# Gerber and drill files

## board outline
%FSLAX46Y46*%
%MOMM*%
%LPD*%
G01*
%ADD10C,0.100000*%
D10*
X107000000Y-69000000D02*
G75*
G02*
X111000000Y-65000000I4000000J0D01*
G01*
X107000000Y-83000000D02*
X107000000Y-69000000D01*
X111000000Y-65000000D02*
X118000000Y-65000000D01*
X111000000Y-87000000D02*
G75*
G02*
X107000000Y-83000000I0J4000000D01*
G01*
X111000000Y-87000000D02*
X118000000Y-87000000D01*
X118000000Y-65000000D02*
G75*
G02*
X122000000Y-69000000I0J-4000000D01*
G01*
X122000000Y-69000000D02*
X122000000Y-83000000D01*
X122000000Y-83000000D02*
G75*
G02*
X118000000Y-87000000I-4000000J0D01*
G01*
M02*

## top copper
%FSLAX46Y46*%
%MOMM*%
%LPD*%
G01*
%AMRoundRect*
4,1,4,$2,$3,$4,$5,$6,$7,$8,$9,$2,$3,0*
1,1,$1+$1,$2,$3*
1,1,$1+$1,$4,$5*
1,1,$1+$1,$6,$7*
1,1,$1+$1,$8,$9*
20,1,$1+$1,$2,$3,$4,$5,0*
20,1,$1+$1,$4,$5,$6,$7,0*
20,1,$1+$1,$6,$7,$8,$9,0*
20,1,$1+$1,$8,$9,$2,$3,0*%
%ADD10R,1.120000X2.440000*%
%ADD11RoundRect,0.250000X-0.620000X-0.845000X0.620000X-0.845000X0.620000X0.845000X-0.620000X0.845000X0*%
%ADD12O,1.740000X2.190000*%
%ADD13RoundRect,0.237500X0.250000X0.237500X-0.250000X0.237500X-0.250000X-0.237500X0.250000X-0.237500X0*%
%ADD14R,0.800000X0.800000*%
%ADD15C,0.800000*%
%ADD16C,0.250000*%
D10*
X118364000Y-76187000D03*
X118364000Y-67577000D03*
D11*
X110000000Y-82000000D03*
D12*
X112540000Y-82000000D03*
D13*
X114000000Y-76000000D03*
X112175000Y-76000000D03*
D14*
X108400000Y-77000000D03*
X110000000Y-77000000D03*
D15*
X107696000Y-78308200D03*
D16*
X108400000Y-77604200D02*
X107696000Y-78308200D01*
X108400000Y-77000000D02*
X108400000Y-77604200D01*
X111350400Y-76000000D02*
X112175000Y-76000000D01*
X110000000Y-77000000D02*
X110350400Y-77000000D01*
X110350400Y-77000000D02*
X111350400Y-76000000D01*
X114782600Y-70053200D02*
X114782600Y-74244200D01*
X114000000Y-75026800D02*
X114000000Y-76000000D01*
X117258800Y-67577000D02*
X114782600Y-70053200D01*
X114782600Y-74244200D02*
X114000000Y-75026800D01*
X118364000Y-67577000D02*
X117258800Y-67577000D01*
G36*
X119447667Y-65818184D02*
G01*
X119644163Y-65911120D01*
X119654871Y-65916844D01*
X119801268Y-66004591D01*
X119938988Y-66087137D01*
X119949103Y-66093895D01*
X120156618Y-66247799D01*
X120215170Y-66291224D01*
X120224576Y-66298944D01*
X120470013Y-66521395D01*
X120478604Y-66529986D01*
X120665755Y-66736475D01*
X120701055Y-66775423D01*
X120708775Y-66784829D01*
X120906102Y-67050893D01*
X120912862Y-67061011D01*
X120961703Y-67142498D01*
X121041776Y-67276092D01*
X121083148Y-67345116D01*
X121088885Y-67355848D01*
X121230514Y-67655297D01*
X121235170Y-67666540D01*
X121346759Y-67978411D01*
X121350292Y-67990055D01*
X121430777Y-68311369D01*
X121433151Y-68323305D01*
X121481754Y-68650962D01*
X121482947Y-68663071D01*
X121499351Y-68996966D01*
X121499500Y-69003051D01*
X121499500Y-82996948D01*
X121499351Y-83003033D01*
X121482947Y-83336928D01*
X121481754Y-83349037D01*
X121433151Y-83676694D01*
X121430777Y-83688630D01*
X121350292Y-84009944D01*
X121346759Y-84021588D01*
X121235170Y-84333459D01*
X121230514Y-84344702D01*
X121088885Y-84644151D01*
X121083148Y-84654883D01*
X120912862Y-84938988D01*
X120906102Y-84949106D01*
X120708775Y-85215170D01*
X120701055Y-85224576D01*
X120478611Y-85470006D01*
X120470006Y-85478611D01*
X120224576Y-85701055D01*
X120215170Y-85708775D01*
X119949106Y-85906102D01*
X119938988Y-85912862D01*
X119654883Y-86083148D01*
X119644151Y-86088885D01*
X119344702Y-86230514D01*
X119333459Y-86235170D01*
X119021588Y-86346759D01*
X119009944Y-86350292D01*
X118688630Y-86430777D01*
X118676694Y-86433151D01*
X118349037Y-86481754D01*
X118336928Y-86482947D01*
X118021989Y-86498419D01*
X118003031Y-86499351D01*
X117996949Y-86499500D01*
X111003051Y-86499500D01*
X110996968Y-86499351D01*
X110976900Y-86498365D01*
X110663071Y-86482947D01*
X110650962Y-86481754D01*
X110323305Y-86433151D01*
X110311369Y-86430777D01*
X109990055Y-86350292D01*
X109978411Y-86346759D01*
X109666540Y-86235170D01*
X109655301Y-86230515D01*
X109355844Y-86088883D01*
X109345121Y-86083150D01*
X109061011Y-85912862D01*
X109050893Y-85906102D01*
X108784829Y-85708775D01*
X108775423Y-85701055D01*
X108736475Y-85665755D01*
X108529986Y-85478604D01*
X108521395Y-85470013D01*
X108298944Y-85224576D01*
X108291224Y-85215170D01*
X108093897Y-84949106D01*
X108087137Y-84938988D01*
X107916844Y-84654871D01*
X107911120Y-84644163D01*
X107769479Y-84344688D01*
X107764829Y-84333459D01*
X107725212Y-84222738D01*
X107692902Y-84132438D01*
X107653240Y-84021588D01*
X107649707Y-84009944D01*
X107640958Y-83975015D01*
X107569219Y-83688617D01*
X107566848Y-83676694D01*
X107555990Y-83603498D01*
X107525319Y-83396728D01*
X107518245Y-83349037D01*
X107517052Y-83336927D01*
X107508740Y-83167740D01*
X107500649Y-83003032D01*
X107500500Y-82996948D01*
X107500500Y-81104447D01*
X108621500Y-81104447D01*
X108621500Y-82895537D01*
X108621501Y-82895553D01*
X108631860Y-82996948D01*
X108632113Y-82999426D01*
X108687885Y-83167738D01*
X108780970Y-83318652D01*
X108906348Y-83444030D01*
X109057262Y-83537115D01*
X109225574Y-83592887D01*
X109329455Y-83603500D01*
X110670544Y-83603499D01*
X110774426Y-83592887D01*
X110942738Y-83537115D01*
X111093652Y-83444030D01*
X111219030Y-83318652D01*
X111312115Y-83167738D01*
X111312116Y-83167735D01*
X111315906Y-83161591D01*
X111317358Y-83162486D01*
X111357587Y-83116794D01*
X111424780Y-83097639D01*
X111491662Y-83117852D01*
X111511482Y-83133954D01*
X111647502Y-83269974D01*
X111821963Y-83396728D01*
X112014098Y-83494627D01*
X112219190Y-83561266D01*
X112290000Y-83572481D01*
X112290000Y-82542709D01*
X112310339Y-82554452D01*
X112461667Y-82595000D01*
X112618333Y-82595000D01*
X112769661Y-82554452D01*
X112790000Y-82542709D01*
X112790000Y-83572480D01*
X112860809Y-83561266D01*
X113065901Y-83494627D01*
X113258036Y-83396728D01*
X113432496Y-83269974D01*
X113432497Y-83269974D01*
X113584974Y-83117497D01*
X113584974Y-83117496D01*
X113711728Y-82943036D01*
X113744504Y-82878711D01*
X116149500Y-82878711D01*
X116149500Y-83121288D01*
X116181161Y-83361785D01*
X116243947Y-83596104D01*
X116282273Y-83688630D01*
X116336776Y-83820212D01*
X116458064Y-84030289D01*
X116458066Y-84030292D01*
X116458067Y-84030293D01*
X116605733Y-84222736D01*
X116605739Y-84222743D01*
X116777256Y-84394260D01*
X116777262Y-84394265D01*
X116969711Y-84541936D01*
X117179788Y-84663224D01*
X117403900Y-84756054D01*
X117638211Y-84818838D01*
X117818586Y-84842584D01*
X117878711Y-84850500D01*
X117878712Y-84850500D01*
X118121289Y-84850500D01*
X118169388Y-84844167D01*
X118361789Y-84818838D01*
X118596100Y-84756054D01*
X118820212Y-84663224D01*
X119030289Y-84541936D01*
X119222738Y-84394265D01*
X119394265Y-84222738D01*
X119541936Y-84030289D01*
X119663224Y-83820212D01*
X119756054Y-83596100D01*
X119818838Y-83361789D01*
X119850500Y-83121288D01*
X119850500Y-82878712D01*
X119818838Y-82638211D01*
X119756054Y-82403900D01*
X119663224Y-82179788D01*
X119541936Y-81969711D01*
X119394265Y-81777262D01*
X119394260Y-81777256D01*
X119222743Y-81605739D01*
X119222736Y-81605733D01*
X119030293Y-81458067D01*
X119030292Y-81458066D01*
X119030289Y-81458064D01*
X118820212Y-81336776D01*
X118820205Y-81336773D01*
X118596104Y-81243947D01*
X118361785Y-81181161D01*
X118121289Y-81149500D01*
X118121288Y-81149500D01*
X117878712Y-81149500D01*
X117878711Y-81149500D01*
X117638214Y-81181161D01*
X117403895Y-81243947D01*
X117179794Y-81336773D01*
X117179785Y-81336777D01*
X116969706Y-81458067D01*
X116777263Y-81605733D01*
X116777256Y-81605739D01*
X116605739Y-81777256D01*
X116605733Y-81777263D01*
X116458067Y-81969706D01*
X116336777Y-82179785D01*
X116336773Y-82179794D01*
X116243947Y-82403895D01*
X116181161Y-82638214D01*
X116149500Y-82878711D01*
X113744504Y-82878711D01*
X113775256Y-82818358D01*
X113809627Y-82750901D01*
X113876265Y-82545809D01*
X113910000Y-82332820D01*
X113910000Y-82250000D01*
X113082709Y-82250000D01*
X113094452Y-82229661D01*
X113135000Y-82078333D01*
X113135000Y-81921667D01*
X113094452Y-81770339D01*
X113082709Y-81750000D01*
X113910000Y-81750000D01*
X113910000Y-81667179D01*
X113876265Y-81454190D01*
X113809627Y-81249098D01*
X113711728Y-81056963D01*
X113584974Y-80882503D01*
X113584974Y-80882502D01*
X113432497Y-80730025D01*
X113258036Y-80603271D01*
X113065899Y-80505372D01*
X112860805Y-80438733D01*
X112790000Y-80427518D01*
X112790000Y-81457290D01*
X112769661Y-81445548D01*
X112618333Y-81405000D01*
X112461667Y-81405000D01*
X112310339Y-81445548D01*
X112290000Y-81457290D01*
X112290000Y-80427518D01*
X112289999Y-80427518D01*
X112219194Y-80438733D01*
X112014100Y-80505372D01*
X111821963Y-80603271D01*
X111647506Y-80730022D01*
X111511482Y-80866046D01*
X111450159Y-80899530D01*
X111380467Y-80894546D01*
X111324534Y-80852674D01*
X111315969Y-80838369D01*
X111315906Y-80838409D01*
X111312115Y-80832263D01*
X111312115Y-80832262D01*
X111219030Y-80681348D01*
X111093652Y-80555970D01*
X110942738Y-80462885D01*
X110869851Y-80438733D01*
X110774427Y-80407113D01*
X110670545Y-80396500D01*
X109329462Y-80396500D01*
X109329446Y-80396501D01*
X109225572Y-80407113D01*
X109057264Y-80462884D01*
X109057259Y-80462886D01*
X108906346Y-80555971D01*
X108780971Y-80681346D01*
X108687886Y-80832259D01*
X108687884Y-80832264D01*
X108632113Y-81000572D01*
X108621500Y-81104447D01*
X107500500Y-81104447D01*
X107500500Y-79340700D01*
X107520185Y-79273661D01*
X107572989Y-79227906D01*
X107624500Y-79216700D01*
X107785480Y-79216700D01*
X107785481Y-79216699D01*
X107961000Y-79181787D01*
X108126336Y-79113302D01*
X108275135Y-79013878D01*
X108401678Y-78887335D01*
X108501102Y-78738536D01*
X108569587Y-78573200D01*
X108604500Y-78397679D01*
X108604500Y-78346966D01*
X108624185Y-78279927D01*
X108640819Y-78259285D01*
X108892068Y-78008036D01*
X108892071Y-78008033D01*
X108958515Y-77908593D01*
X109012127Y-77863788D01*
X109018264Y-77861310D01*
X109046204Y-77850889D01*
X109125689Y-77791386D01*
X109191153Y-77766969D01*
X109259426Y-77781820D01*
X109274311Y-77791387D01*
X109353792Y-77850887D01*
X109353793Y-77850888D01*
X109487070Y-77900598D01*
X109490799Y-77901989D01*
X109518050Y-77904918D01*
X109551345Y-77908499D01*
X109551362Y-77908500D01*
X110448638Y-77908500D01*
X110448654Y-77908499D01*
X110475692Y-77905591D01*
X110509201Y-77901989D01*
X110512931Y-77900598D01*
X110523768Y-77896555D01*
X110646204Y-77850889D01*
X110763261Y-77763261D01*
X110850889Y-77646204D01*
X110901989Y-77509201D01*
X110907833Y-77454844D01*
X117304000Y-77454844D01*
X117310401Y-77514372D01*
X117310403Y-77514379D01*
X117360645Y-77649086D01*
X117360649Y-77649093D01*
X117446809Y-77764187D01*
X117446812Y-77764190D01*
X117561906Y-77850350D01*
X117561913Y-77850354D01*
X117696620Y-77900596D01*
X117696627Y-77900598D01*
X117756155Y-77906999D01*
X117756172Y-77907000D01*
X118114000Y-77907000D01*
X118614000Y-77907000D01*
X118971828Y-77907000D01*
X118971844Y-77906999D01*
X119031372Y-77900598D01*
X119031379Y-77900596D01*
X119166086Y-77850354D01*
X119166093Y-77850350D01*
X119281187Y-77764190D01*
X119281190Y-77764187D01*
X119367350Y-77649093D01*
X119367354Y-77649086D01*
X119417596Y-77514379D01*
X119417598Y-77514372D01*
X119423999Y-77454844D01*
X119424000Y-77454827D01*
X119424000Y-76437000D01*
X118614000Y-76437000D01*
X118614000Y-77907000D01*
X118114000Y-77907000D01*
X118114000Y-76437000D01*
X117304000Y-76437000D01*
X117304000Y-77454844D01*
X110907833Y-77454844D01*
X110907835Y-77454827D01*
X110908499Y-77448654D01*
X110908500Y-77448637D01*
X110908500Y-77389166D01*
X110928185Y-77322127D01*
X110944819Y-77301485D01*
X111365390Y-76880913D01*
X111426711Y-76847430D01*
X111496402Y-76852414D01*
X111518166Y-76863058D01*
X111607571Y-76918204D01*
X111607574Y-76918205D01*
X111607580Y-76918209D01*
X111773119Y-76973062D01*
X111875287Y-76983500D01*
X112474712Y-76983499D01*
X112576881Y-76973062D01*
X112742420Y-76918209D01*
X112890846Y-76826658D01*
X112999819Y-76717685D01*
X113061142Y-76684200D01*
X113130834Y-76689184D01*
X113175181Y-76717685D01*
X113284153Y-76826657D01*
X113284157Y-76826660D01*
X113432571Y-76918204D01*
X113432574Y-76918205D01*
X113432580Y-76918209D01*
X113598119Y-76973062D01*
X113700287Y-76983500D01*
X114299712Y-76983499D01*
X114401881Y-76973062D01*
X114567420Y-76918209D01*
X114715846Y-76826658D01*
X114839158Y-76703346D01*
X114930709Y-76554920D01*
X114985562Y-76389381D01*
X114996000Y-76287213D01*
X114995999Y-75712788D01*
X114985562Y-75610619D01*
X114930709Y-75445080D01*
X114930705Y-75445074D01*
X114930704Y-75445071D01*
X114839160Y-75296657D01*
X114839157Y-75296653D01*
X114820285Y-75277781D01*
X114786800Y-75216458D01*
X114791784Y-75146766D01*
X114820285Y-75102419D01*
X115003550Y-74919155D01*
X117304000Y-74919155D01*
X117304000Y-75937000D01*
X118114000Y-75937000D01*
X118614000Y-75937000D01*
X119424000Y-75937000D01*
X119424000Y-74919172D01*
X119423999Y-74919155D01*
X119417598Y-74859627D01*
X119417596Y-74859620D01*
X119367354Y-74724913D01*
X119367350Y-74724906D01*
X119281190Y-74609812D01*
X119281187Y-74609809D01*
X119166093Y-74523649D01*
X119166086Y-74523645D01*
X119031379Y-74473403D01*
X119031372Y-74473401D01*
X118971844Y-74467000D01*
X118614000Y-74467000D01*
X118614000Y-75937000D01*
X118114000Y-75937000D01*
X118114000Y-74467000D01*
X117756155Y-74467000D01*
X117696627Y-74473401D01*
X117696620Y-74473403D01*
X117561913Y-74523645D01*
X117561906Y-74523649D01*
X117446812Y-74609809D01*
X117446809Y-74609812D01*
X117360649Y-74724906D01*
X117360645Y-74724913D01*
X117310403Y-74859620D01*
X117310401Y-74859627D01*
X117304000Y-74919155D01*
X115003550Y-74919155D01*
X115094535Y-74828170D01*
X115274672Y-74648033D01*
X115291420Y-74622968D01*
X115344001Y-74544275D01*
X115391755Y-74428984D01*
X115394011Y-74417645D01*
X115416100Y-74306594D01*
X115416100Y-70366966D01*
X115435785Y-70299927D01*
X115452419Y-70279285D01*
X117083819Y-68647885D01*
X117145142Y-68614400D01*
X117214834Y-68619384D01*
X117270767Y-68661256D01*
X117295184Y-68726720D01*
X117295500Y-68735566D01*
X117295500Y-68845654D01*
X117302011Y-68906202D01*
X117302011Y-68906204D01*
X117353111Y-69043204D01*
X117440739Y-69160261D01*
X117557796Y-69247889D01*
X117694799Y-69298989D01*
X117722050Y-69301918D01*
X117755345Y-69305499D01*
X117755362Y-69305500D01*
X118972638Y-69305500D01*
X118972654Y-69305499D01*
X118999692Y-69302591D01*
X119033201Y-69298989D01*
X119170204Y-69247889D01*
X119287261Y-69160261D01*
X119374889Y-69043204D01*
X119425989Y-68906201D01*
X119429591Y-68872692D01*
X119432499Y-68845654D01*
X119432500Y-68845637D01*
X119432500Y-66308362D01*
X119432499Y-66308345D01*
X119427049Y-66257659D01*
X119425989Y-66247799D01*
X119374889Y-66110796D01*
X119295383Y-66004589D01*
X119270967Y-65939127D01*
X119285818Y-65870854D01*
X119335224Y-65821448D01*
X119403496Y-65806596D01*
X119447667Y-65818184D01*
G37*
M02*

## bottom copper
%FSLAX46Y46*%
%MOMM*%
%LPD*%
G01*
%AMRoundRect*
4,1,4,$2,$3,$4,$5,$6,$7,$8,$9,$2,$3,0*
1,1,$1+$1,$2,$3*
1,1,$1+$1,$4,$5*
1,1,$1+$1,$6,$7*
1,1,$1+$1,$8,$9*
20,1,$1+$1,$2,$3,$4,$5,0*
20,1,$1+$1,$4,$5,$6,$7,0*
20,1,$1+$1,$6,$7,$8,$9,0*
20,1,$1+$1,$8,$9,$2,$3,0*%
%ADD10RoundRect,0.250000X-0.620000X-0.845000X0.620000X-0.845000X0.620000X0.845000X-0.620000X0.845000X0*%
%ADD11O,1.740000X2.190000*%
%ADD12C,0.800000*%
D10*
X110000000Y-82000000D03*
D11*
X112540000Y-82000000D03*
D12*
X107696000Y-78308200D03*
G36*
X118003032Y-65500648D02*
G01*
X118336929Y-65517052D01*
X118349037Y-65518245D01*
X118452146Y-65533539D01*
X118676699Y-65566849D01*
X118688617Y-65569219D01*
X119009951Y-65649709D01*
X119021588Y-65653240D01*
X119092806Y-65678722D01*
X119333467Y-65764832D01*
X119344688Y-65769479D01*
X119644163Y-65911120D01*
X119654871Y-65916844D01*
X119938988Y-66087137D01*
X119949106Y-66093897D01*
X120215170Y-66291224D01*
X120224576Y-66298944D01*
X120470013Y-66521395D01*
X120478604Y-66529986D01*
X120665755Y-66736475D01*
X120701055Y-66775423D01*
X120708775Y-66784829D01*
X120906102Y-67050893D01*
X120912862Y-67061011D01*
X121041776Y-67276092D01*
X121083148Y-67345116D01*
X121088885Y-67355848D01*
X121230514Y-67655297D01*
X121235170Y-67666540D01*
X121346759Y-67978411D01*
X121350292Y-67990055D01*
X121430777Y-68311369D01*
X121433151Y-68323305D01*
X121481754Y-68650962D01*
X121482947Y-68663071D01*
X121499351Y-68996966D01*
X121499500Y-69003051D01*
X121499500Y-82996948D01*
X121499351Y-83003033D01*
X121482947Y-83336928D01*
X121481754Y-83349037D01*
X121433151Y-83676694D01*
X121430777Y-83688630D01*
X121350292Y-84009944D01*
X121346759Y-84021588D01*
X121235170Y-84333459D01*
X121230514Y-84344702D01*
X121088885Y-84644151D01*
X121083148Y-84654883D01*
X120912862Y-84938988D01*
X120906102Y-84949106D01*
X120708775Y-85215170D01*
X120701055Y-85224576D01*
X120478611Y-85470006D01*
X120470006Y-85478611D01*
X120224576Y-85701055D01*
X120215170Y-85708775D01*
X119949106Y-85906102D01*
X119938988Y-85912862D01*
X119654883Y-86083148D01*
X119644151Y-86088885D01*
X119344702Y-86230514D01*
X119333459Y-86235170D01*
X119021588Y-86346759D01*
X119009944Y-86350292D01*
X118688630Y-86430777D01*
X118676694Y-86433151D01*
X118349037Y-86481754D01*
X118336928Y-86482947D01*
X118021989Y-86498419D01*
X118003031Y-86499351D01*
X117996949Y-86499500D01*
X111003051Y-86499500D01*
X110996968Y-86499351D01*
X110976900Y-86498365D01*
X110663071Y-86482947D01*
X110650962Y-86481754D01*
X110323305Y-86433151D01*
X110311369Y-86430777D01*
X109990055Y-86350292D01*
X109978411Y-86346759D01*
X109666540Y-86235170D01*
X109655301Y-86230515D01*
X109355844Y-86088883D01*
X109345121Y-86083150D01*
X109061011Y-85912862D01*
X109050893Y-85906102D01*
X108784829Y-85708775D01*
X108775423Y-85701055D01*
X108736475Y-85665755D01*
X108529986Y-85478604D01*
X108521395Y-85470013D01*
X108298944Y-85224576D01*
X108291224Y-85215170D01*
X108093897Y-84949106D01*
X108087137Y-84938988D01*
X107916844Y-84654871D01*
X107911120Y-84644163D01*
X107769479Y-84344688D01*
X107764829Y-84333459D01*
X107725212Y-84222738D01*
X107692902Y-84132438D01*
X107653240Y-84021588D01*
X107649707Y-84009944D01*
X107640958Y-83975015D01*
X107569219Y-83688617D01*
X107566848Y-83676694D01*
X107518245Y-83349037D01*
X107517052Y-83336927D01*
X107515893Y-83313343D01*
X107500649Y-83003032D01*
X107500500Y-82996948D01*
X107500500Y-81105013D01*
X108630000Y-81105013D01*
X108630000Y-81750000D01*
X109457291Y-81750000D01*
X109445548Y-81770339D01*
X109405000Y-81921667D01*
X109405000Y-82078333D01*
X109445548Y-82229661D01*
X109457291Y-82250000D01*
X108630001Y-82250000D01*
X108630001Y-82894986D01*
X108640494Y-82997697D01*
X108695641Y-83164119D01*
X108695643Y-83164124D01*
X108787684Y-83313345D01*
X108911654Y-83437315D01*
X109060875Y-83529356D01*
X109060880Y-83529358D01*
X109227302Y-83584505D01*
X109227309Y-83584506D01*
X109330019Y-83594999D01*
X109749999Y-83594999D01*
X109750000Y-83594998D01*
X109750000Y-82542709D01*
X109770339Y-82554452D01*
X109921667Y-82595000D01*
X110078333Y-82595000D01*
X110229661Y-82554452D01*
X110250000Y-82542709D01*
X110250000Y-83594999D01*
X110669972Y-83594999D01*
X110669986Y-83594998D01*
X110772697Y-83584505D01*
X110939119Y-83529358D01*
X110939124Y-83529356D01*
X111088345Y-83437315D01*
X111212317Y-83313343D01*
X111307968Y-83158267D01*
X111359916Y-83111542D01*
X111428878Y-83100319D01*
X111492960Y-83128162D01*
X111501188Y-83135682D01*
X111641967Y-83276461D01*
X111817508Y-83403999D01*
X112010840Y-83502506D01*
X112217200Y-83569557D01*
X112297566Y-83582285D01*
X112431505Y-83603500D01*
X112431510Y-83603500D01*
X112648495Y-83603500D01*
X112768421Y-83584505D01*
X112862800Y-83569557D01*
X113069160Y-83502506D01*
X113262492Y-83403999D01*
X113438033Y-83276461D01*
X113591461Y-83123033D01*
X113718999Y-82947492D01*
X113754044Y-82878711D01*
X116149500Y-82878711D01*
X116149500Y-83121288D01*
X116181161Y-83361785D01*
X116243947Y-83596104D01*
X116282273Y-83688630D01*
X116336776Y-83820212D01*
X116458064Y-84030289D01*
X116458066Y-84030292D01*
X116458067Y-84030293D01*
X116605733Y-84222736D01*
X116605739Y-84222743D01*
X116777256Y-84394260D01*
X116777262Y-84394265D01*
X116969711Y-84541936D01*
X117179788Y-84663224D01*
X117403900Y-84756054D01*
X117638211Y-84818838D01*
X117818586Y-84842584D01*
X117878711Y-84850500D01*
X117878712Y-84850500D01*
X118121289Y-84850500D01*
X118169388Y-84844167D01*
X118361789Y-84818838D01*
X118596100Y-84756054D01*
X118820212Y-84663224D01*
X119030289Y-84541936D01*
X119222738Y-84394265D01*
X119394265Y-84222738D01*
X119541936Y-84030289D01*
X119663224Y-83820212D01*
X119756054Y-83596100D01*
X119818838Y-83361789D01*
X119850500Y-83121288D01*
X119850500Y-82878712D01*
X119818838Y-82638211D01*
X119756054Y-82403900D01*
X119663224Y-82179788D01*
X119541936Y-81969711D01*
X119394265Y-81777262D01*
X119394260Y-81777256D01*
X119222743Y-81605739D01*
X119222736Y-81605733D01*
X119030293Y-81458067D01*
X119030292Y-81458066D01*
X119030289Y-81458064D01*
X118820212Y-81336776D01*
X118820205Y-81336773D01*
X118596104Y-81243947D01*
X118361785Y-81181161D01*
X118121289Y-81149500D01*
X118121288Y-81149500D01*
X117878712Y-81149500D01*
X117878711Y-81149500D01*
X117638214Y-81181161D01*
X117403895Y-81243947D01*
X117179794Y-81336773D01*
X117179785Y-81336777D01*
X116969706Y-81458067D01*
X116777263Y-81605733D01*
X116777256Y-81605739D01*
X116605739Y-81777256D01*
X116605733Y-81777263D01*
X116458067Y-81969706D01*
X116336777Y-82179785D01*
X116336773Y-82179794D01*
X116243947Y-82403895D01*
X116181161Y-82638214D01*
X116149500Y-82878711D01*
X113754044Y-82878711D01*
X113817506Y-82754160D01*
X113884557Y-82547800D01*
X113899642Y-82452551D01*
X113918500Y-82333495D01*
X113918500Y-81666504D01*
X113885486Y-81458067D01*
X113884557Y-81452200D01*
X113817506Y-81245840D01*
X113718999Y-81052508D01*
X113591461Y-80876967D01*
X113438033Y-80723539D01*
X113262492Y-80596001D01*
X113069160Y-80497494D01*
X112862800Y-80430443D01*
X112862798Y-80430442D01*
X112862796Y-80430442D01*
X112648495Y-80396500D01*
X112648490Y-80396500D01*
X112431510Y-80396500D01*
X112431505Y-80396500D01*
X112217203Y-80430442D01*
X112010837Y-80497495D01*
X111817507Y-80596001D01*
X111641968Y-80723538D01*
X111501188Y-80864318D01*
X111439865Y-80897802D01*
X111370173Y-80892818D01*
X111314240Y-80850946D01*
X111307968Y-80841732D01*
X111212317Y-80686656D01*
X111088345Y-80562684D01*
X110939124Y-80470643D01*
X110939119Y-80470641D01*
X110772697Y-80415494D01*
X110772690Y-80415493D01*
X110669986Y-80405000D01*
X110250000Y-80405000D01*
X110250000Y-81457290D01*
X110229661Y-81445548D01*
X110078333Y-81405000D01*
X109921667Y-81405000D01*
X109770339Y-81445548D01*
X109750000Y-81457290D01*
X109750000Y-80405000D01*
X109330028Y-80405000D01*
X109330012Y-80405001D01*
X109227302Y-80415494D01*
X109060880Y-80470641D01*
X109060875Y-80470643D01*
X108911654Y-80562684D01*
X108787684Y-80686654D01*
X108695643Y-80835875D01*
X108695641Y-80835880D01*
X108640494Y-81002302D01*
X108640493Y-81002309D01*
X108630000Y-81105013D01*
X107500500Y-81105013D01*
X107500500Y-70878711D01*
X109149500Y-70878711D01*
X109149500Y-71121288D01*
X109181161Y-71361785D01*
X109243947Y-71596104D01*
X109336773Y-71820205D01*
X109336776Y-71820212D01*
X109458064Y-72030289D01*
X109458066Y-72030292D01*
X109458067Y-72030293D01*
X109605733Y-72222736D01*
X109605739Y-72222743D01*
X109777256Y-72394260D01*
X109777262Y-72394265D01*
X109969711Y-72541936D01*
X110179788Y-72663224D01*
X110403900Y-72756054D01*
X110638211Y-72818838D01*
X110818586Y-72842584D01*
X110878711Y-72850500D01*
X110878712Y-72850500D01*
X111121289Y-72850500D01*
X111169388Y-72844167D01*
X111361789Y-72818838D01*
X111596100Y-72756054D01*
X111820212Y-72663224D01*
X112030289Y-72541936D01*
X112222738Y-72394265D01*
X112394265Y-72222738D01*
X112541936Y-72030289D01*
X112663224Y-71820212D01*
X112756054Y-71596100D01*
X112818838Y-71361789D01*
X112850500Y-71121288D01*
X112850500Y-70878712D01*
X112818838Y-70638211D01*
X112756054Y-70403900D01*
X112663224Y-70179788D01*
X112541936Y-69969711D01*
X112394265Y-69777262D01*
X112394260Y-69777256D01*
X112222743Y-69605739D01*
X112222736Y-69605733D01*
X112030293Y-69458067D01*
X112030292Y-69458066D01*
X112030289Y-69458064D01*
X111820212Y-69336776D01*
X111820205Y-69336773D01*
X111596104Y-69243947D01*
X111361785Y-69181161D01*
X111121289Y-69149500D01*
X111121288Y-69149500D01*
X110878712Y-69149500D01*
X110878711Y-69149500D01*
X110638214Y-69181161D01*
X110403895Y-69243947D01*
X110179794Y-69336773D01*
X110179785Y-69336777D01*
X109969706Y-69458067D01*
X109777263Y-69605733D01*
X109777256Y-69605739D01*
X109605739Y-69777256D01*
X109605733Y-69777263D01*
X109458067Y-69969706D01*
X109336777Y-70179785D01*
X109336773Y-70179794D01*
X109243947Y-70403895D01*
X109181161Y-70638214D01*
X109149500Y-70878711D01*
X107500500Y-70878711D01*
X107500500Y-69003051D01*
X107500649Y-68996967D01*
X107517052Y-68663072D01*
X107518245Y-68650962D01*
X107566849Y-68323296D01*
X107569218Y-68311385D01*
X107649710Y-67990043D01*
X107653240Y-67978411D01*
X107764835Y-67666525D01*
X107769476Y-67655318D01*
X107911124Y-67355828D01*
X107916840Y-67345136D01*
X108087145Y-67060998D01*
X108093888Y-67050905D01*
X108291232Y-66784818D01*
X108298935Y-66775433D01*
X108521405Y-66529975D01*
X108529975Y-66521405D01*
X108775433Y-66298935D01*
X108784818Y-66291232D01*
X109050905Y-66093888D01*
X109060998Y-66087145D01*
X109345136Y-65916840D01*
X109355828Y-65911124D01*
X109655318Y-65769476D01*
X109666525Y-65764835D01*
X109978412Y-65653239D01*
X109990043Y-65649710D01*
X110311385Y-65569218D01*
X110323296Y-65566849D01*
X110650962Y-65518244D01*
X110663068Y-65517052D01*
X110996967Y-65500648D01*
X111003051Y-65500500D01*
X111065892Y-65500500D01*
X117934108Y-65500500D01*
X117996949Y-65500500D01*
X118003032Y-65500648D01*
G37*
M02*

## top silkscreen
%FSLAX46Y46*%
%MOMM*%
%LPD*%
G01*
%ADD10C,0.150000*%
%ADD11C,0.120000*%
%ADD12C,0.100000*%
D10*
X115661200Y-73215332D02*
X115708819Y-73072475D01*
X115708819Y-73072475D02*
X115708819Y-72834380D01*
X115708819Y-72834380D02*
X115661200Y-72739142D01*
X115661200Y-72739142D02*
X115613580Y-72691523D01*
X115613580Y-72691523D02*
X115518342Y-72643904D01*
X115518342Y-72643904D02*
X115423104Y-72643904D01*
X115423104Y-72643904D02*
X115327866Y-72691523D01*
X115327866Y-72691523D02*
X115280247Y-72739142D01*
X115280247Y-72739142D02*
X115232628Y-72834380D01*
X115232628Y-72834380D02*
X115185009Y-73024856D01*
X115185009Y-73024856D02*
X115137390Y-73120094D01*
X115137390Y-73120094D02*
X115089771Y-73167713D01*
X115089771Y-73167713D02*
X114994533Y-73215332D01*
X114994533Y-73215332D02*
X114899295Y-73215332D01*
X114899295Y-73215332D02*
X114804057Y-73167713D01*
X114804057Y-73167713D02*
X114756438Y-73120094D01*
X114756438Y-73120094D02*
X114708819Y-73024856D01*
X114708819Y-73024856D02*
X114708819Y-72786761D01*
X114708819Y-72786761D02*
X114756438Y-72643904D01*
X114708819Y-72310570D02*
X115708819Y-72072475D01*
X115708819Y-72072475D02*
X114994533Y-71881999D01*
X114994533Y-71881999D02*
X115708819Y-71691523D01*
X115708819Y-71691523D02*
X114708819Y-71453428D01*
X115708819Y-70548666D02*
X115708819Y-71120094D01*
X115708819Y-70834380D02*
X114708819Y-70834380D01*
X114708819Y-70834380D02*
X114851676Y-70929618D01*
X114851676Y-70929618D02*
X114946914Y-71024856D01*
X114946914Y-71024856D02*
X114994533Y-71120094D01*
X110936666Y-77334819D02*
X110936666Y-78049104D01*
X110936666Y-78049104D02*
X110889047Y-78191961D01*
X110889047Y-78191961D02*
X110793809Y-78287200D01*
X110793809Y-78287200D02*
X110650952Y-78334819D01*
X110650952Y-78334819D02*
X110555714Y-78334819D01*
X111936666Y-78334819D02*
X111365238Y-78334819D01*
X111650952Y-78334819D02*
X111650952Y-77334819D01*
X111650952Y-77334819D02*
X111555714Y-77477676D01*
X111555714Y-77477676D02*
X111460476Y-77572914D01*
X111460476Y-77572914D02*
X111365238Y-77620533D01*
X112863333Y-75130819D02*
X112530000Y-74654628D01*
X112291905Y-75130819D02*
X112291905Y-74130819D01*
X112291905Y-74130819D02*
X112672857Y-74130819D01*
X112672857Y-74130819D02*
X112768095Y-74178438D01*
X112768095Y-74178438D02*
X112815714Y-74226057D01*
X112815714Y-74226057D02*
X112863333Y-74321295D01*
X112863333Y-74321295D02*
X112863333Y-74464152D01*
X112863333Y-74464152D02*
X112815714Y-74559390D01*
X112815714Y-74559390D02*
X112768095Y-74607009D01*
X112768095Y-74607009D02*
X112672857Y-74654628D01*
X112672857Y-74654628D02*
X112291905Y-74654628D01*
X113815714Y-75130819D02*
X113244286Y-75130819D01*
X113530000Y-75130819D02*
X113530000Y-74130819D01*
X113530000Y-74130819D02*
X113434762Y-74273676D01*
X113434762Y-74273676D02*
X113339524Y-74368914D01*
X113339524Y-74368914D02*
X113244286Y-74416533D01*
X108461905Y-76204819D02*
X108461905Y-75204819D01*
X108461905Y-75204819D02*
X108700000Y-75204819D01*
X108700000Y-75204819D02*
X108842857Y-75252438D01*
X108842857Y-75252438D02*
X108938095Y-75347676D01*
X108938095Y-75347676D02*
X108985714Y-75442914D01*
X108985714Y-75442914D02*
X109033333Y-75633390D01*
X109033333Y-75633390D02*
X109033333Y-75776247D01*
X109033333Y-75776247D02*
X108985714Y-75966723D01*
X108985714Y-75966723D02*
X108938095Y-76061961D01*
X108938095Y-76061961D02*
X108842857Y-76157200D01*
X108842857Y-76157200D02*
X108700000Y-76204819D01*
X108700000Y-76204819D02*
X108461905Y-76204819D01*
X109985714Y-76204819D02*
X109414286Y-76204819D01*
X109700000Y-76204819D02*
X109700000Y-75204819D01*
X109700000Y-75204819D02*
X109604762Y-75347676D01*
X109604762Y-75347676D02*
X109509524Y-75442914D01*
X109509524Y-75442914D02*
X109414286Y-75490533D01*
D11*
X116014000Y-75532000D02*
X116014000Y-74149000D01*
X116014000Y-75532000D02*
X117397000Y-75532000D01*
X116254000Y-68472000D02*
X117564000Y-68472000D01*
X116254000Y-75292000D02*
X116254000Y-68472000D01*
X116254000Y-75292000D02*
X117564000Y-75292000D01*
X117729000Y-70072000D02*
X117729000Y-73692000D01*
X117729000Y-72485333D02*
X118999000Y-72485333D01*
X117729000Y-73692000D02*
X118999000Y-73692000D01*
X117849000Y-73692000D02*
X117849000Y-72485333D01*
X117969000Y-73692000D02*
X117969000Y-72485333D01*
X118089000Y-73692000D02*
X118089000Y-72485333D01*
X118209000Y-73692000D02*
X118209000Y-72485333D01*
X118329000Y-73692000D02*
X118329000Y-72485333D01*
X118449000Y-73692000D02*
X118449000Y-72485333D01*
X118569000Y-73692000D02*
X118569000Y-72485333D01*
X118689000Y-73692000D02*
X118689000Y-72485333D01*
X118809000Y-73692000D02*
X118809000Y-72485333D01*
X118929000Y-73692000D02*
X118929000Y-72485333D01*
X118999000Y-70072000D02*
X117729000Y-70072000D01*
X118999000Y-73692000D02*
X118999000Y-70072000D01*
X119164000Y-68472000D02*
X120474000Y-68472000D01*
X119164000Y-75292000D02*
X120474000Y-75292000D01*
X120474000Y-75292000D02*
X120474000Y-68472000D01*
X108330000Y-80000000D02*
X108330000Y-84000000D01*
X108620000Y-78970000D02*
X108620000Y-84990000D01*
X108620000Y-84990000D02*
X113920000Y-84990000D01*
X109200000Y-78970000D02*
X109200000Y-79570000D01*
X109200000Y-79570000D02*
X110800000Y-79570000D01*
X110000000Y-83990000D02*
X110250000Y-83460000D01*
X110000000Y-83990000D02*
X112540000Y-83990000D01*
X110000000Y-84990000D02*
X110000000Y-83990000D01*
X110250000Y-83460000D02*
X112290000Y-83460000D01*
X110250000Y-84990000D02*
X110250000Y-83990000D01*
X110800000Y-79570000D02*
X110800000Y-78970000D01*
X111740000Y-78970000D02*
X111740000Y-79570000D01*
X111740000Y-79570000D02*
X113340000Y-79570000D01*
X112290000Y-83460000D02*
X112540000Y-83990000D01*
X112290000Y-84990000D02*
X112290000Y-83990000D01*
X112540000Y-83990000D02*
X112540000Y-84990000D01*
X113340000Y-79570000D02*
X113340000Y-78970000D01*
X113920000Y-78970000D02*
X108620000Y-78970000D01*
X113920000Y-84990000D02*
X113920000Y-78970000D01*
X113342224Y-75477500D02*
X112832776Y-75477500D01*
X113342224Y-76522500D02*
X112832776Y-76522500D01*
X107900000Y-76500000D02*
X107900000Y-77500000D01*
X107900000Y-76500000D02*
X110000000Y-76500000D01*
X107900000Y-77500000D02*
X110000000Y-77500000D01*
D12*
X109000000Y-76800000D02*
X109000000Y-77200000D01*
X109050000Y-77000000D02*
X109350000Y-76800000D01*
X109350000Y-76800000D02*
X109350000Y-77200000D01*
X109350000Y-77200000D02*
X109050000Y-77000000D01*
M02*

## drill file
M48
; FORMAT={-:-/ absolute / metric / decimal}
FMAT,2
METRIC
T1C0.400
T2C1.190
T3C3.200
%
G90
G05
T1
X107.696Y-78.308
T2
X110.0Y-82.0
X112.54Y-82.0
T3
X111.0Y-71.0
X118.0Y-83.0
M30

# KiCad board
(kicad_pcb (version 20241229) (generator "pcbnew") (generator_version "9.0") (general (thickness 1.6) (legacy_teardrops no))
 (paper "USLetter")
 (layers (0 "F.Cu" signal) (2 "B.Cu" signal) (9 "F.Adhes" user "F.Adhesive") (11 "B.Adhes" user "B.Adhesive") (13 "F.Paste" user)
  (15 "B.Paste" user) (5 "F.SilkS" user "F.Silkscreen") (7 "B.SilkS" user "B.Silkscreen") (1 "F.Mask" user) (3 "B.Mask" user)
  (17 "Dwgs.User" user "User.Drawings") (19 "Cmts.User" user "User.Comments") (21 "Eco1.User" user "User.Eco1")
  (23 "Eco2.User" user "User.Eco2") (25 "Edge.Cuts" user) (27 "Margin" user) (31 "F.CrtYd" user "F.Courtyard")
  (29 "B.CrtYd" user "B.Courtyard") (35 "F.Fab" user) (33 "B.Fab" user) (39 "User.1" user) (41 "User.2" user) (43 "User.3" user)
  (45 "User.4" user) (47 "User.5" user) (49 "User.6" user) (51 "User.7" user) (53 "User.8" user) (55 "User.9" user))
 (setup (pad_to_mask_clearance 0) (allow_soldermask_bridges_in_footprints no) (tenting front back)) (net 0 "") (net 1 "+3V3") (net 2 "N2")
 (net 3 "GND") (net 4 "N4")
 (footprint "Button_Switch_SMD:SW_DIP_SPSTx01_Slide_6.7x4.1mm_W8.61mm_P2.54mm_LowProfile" (layer "F.Cu") (at 118.364 71.882 90)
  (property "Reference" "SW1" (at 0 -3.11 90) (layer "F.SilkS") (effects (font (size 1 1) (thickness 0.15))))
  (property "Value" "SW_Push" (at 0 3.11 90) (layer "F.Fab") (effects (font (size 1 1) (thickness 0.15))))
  (fp_line (start -3.65 -2.35) (end -2.267 -2.35) (stroke (width 0.12) (type solid)) (layer "F.SilkS"))
  (fp_line (start -3.65 -2.35) (end -3.65 -0.967) (stroke (width 0.12) (type solid)) (layer "F.SilkS"))
  (fp_line (start 3.41 -2.11) (end 3.41 -0.8) (stroke (width 0.12) (type solid)) (layer "F.SilkS"))
  (fp_line (start -3.41 -2.11) (end 3.41 -2.11) (stroke (width 0.12) (type solid)) (layer "F.SilkS"))
  (fp_line (start -3.41 -2.11) (end -3.41 -0.8) (stroke (width 0.12) (type solid)) (layer "F.SilkS"))
  (fp_line (start 1.81 -0.635) (end -1.81 -0.635) (stroke (width 0.12) (type solid)) (layer "F.SilkS"))
  (fp_line (start -0.603333 -0.635) (end -0.603333 0.635) (stroke (width 0.12) (type solid)) (layer "F.SilkS"))
  (fp_line (start -1.81 -0.635) (end -1.81 0.635) (stroke (width 0.12) (type solid)) (layer "F.SilkS"))
  (fp_line (start -1.81 -0.515) (end -0.603333 -0.515) (stroke (width 0.12) (type solid)) (layer "F.SilkS"))
  (fp_line (start -1.81 -0.395) (end -0.603333 -0.395) (stroke (width 0.12) (type solid)) (layer "F.SilkS"))
  (fp_line (start -1.81 -0.275) (end -0.603333 -0.275) (stroke (width 0.12) (type solid)) (layer "F.SilkS"))
  (fp_line (start -1.81 -0.155) (end -0.603333 -0.155) (stroke (width 0.12) (type solid)) (layer "F.SilkS"))
  (fp_line (start -1.81 -0.035) (end -0.603333 -0.035) (stroke (width 0.12) (type solid)) (layer "F.SilkS"))
  (fp_line (start -1.81 0.085) (end -0.603333 0.085) (stroke (width 0.12) (type solid)) (layer "F.SilkS"))
  (fp_line (start -1.81 0.205) (end -0.603333 0.205) (stroke (width 0.12) (type solid)) (layer "F.SilkS"))
  (fp_line (start -1.81 0.325) (end -0.603333 0.325) (stroke (width 0.12) (type solid)) (layer "F.SilkS"))
  (fp_line (start -1.81 0.445) (end -0.603333 0.445) (stroke (width 0.12) (type solid)) (layer "F.SilkS"))
  (fp_line (start -1.81 0.565) (end -0.603333 0.565) (stroke (width 0.12) (type solid)) (layer "F.SilkS"))
  (fp_line (start 1.81 0.635) (end 1.81 -0.635) (stroke (width 0.12) (type solid)) (layer "F.SilkS"))
  (fp_line (start -1.81 0.635) (end 1.81 0.635) (stroke (width 0.12) (type solid)) (layer "F.SilkS"))
  (fp_line (start 3.41 0.8) (end 3.41 2.11) (stroke (width 0.12) (type solid)) (layer "F.SilkS"))
  (fp_line (start -3.41 0.8) (end -3.41 2.11) (stroke (width 0.12) (type solid)) (layer "F.SilkS"))
  (fp_line (start -3.41 2.11) (end 3.41 2.11) (stroke (width 0.12) (type solid)) (layer "F.SilkS"))
  (pad "1" smd rect (at -4.305 0 90) (size 2.44 1.12) (layers "F.Cu" "F.Mask" "F.Paste") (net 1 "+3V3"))
  (pad "2" smd rect (at 4.305 0 90) (size 2.44 1.12) (layers "F.Cu" "F.Mask" "F.Paste") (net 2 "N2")))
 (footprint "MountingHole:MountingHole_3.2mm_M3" (layer "F.Cu") (at 118 83)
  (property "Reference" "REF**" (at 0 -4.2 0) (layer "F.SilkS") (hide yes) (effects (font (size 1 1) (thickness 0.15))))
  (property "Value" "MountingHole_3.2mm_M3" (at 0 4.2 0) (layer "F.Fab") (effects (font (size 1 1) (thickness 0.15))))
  (pad "" np_thru_hole circle (at 0 0) (size 3.2 3.2) (drill 3.2) (layers "*.Cu" "*.Mask")))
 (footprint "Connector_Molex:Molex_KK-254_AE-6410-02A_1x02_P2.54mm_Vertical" (layer "F.Cu") (at 110 82)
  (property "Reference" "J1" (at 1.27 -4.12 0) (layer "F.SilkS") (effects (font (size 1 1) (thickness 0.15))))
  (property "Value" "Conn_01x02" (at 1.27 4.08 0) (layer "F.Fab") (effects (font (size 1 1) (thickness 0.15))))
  (fp_line (start -1.67 -2) (end -1.67 2) (stroke (width 0.12) (type solid)) (layer "F.SilkS"))
  (fp_line (start -1.38 -3.03) (end -1.38 2.99) (stroke (width 0.12) (type solid)) (layer "F.SilkS"))
  (fp_line (start -1.38 2.99) (end 3.92 2.99) (stroke (width 0.12) (type solid)) (layer "F.SilkS"))
  (fp_line (start -0.8 -3.03) (end -0.8 -2.43) (stroke (width 0.12) (type solid)) (layer "F.SilkS"))
  (fp_line (start -0.8 -2.43) (end 0.8 -2.43) (stroke (width 0.12) (type solid)) (layer "F.SilkS"))
  (fp_line (start 0 1.99) (end 0.25 1.46) (stroke (width 0.12) (type solid)) (layer "F.SilkS"))
  (fp_line (start 0 1.99) (end 2.54 1.99) (stroke (width 0.12) (type solid)) (layer "F.SilkS"))
  (fp_line (start 0 2.99) (end 0 1.99) (stroke (width 0.12) (type solid)) (layer "F.SilkS"))
  (fp_line (start 0.25 1.46) (end 2.29 1.46) (stroke (width 0.12) (type solid)) (layer "F.SilkS"))
  (fp_line (start 0.25 2.99) (end 0.25 1.99) (stroke (width 0.12) (type solid)) (layer "F.SilkS"))
  (fp_line (start 0.8 -2.43) (end 0.8 -3.03) (stroke (width 0.12) (type solid)) (layer "F.SilkS"))
  (fp_line (start 1.74 -3.03) (end 1.74 -2.43) (stroke (width 0.12) (type solid)) (layer "F.SilkS"))
  (fp_line (start 1.74 -2.43) (end 3.34 -2.43) (stroke (width 0.12) (type solid)) (layer "F.SilkS"))
  (fp_line (start 2.29 1.46) (end 2.54 1.99) (stroke (width 0.12) (type solid)) (layer "F.SilkS"))
  (fp_line (start 2.29 2.99) (end 2.29 1.99) (stroke (width 0.12) (type solid)) (layer "F.SilkS"))
  (fp_line (start 2.54 1.99) (end 2.54 2.99) (stroke (width 0.12) (type solid)) (layer "F.SilkS"))
  (fp_line (start 3.34 -2.43) (end 3.34 -3.03) (stroke (width 0.12) (type solid)) (layer "F.SilkS"))
  (fp_line (start 3.92 -3.03) (end -1.38 -3.03) (stroke (width 0.12) (type solid)) (layer "F.SilkS"))
  (fp_line (start 3.92 2.99) (end 3.92 -3.03) (stroke (width 0.12) (type solid)) (layer "F.SilkS"))
  (pad "1" thru_hole roundrect (at 0 0) (size 1.74 2.19) (drill 1.19) (layers "*.Cu" "*.Mask") (remove_unused_layers no)
   (roundrect_rratio 0.143678) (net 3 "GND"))
  (pad "2" thru_hole oval (at 2.54 0) (size 1.74 2.19) (drill 1.19) (layers "*.Cu" "*.Mask") (remove_unused_layers no) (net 1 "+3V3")))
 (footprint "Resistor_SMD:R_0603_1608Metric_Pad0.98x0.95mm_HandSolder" (layer "F.Cu") (at 113.0875 76 180)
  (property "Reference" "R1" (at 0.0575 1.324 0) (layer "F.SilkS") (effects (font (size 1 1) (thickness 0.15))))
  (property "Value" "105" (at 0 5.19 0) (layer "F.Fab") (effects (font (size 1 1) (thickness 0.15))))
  (fp_line (start -0.254724 0.5225) (end 0.254724 0.5225) (stroke (width 0.12) (type solid)) (layer "F.SilkS"))
  (fp_line (start -0.254724 -0.5225) (end 0.254724 -0.5225) (stroke (width 0.12) (type solid)) (layer "F.SilkS"))
  (pad "1" smd roundrect (at -0.9125 0 180) (size 0.975 0.95) (layers "F.Cu" "F.Mask" "F.Paste") (roundrect_rratio 0.25) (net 2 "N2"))
  (pad "2" smd roundrect (at 0.9125 0 180) (size 0.975 0.95) (layers "F.Cu" "F.Mask" "F.Paste") (roundrect_rratio 0.25) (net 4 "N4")))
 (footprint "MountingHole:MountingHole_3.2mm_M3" (layer "F.Cu") (at 111 71)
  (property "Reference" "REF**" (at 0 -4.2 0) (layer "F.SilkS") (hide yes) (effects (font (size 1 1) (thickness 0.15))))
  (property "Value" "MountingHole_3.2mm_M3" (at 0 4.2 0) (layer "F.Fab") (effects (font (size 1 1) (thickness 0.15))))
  (pad "" np_thru_hole circle (at 0 0) (size 3.2 3.2) (drill 3.2) (layers "*.Cu" "*.Mask")))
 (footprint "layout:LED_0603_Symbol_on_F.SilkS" (layer "F.Cu") (at 109.2 77)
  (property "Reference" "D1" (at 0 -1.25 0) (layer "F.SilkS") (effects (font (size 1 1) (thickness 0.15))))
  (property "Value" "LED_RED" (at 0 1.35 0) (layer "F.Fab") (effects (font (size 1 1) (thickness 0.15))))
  (fp_line (start -1.3 -0.5) (end -1.3 0.5) (stroke (width 0.12) (type solid)) (layer "F.SilkS"))
  (fp_line (start -1.3 -0.5) (end 0.8 -0.5) (stroke (width 0.12) (type solid)) (layer "F.SilkS"))
  (fp_line (start -1.3 0.5) (end 0.8 0.5) (stroke (width 0.12) (type solid)) (layer "F.SilkS"))
  (fp_line (start -0.2 -0.2) (end -0.2 0.2) (stroke (width 0.1) (type solid)) (layer "F.SilkS"))
  (fp_line (start -0.15 0) (end 0.15 -0.2) (stroke (width 0.1) (type solid)) (layer "F.SilkS"))
  (fp_line (start 0.15 -0.2) (end 0.15 0.2) (stroke (width 0.1) (type solid)) (layer "F.SilkS"))
  (fp_line (start 0.15 0.2) (end -0.15 0) (stroke (width 0.1) (type solid)) (layer "F.SilkS"))
  (pad "1" smd rect (at -0.8 0 180) (size 0.8 0.8) (layers "F.Cu" "F.Mask" "F.Paste") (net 3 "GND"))
  (pad "2" smd rect (at 0.8 0 180) (size 0.8 0.8) (layers "F.Cu" "F.Mask" "F.Paste") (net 4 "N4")))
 (gr_arc (start 107 69) (mid 108.171573 66.171573) (end 111 65) (stroke (width 0.1) (type default)) (layer "Edge.Cuts"))
 (gr_line (start 107 83) (end 107 69) (stroke (width 0.1) (type default)) (layer "Edge.Cuts"))
 (gr_line (start 111 65) (end 118 65) (stroke (width 0.1) (type default)) (layer "Edge.Cuts"))
 (gr_arc (start 111 87) (mid 108.171573 85.828427) (end 107 83) (stroke (width 0.1) (type default)) (layer "Edge.Cuts"))
 (gr_line (start 111 87) (end 118 87) (stroke (width 0.1) (type default)) (layer "Edge.Cuts"))
 (gr_arc (start 118 65) (mid 120.828427 66.171573) (end 122 69) (stroke (width 0.1) (type default)) (layer "Edge.Cuts"))
 (gr_line (start 122 69) (end 122 83) (stroke (width 0.1) (type default)) (layer "Edge.Cuts"))
 (gr_arc (start 122 83) (mid 120.828427 85.828427) (end 118 87) (stroke (width 0.1) (type default)) (layer "Edge.Cuts"))
 (segment (start 108.4 77.6042) (end 107.696 78.3082) (width 0.25) (layer "F.Cu") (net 3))
 (segment (start 108.4 77) (end 108.4 77.6042) (width 0.25) (layer "F.Cu") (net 3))
 (via (at 107.696 78.3082) (size 0.8) (drill 0.4) (layers "F.Cu" "B.Cu") (free yes) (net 3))
 (segment (start 111.3504 76) (end 112.175 76) (width 0.25) (layer "F.Cu") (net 4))
 (segment (start 110 77) (end 110.3504 77) (width 0.25) (layer "F.Cu") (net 4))
 (segment (start 110.3504 77) (end 111.3504 76) (width 0.25) (layer "F.Cu") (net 4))
 (segment (start 114.7826 70.0532) (end 114.7826 74.2442) (width 0.25) (layer "F.Cu") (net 2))
 (segment (start 114 75.0268) (end 114 76) (width 0.25) (layer "F.Cu") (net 2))
 (segment (start 117.2588 67.577) (end 114.7826 70.0532) (width 0.25) (layer "F.Cu") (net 2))
 (segment (start 114.7826 74.2442) (end 114 75.0268) (width 0.25) (layer "F.Cu") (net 2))
 (segment (start 118.364 67.577) (end 117.2588 67.577) (width 0.25) (layer "F.Cu") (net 2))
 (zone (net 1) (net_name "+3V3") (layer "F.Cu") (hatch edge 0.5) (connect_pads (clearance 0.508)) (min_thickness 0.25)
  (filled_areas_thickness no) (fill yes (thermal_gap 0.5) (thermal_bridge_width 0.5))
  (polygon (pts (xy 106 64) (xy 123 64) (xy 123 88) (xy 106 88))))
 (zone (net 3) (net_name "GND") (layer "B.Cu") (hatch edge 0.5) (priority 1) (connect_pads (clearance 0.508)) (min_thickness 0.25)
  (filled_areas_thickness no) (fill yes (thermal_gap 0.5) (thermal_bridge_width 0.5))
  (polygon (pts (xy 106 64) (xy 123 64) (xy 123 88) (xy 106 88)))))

